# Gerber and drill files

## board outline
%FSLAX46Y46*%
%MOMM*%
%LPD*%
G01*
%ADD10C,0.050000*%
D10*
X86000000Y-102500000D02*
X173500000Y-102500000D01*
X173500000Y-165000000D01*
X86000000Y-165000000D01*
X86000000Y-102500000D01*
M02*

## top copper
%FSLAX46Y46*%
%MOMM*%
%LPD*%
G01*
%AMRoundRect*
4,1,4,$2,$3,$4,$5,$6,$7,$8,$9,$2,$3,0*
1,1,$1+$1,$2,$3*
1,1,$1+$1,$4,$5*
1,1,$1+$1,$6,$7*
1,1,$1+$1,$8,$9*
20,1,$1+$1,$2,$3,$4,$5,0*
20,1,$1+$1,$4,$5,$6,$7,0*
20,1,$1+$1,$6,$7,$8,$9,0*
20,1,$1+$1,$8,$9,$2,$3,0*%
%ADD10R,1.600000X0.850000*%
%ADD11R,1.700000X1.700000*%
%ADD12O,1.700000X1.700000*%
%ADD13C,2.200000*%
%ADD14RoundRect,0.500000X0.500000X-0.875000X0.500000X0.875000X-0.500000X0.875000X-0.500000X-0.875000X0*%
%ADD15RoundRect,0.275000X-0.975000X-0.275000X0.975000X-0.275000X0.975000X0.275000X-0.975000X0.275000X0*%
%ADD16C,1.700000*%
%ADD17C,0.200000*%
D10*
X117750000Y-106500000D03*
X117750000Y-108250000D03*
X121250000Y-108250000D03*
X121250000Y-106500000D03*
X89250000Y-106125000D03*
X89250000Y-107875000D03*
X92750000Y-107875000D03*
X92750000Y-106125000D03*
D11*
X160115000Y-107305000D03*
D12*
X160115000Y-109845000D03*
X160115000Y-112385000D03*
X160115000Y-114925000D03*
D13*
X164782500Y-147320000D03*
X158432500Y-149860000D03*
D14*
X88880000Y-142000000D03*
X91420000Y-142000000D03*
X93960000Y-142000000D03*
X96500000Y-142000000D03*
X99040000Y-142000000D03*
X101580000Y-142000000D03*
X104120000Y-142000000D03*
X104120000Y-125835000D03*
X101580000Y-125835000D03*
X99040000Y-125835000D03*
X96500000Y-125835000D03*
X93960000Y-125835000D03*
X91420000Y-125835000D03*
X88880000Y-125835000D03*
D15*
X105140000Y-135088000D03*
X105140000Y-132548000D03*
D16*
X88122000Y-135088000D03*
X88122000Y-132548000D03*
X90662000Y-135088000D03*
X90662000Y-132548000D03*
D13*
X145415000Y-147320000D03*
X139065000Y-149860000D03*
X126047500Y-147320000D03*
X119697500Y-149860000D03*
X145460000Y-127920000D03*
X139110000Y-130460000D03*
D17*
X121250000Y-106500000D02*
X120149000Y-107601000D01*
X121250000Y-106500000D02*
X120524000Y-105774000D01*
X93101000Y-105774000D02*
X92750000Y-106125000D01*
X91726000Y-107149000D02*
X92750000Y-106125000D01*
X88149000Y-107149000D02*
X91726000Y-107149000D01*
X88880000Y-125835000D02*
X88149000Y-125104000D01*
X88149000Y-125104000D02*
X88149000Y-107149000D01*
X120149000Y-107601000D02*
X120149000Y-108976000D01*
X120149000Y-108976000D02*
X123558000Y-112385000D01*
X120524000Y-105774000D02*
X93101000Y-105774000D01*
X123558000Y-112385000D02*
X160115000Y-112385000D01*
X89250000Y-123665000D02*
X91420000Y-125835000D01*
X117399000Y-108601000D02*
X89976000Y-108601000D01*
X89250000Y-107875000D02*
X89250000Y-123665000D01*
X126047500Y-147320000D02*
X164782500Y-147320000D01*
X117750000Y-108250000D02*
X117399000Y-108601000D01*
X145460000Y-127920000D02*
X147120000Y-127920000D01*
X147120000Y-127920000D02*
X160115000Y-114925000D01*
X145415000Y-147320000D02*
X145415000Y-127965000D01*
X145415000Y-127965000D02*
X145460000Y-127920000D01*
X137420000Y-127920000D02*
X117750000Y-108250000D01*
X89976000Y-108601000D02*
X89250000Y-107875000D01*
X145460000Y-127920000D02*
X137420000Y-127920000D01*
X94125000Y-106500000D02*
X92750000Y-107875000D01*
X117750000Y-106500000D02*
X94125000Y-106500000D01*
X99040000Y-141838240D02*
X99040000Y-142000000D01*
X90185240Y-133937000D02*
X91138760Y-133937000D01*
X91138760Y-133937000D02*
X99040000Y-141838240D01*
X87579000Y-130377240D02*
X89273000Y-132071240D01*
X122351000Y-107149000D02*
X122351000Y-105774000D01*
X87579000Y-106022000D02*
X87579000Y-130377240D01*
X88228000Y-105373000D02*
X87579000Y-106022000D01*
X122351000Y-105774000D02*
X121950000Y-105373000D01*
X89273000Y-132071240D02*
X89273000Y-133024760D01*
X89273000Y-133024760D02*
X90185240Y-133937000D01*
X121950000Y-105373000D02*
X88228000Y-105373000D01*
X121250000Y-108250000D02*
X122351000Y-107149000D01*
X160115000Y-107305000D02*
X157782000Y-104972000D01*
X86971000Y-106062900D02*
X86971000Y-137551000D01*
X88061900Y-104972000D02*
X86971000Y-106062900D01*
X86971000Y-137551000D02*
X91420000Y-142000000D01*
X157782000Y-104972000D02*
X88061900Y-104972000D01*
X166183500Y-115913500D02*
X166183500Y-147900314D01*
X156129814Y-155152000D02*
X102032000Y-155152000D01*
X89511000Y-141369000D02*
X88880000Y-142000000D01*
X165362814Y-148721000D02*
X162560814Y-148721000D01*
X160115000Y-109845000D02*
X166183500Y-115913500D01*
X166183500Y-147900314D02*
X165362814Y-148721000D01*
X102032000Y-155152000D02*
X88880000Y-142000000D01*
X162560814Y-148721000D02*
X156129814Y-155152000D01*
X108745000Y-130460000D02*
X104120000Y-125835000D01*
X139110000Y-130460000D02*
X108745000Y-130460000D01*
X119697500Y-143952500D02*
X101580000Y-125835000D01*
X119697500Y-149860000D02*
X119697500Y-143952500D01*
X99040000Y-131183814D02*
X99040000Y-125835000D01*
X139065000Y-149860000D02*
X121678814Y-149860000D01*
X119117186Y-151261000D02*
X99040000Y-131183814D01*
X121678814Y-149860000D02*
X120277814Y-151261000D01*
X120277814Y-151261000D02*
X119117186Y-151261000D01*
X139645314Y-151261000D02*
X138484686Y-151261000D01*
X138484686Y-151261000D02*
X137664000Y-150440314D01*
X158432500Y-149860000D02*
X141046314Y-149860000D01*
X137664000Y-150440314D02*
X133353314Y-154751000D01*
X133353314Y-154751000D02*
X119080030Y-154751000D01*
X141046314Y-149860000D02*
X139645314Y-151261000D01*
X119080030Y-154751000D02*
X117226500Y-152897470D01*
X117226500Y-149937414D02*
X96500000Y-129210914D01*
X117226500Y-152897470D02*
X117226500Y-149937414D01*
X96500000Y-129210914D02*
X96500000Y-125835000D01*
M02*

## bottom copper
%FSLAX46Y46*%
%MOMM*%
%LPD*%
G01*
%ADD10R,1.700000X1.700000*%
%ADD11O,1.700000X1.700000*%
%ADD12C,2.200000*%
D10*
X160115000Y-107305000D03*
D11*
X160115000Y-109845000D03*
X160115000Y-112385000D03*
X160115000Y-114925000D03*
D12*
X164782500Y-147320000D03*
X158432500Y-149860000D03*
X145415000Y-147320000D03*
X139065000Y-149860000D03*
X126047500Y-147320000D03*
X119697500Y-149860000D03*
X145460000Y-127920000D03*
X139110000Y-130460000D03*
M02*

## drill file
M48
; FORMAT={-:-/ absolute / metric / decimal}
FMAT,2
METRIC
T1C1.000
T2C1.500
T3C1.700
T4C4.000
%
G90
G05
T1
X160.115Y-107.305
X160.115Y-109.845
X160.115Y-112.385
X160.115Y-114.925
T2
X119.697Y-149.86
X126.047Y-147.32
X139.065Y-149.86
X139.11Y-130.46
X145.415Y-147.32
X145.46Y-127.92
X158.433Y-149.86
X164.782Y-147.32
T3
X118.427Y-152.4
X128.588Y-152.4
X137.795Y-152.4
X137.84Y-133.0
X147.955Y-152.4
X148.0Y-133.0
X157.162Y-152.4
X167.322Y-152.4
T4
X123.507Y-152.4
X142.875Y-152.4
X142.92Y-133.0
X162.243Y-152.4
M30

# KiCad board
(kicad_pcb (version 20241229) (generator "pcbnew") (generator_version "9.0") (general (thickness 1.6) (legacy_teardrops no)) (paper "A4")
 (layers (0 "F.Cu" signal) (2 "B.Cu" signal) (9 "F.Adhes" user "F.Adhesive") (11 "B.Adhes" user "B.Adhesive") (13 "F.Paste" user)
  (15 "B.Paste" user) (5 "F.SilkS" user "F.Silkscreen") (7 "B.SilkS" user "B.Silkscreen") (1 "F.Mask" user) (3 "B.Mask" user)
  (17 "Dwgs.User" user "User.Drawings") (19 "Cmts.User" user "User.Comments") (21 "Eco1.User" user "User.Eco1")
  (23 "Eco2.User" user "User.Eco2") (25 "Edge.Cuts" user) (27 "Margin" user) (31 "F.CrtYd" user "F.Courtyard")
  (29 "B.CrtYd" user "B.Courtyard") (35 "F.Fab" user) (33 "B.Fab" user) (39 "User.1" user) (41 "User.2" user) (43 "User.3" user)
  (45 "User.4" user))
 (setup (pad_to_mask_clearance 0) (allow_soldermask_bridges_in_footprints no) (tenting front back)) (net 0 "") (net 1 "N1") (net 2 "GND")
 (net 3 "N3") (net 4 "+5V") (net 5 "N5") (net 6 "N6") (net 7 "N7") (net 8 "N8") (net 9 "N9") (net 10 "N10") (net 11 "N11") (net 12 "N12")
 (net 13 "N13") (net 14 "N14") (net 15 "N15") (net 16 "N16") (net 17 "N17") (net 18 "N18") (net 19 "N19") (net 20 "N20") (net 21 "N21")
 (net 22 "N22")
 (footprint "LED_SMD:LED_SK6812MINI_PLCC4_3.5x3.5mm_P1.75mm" (layer "F.Cu") (at 119.5 107.375)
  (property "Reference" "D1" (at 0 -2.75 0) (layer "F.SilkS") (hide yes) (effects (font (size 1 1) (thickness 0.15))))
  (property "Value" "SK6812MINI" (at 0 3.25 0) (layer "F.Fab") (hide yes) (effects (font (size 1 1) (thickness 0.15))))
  (pad "1" smd rect (at -1.75 -0.875) (size 1.6 0.85) (layers "F.Cu" "F.Mask" "F.Paste") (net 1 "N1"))
  (pad "2" smd rect (at -1.75 0.875) (size 1.6 0.85) (layers "F.Cu" "F.Mask" "F.Paste") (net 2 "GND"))
  (pad "3" smd rect (at 1.75 0.875) (size 1.6 0.85) (layers "F.Cu" "F.Mask" "F.Paste") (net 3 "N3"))
  (pad "4" smd rect (at 1.75 -0.875) (size 1.6 0.85) (layers "F.Cu" "F.Mask" "F.Paste") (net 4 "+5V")))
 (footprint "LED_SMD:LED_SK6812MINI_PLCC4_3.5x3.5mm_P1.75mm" (layer "F.Cu") (at 91 107)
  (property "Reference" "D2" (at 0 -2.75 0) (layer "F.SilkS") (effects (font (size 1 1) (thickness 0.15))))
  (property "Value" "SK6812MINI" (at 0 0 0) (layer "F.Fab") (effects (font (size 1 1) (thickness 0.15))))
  (pad "1" smd rect (at -1.75 -0.875) (size 1.6 0.85) (layers "F.Cu" "F.Mask" "F.Paste") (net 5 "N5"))
  (pad "2" smd rect (at -1.75 0.875) (size 1.6 0.85) (layers "F.Cu" "F.Mask" "F.Paste") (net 2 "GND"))
  (pad "3" smd rect (at 1.75 0.875) (size 1.6 0.85) (layers "F.Cu" "F.Mask" "F.Paste") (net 1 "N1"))
  (pad "4" smd rect (at 1.75 -0.875) (size 1.6 0.85) (layers "F.Cu" "F.Mask" "F.Paste") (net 4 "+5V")))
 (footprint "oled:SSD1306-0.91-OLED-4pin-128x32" (layer "F.Cu") (at 123.615 105.115)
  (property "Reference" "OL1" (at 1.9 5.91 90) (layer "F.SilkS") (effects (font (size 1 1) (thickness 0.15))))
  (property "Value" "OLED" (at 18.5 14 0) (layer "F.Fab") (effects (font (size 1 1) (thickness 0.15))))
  (pad "1" thru_hole rect (at 36.5 2.19) (size 1.7 1.7) (drill 1) (layers "*.Cu" "*.Mask") (remove_unused_layers no) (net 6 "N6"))
  (pad "2" thru_hole oval (at 36.5 4.73) (size 1.7 1.7) (drill 1) (layers "*.Cu" "*.Mask") (remove_unused_layers no) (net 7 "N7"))
  (pad "3" thru_hole oval (at 36.5 7.27) (size 1.7 1.7) (drill 1) (layers "*.Cu" "*.Mask") (remove_unused_layers no) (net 4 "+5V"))
  (pad "4" thru_hole oval (at 36.5 9.81) (size 1.7 1.7) (drill 1) (layers "*.Cu" "*.Mask") (remove_unused_layers no) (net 2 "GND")))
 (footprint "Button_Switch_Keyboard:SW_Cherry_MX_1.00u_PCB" (layer "F.Cu") (at 164.7825 147.32)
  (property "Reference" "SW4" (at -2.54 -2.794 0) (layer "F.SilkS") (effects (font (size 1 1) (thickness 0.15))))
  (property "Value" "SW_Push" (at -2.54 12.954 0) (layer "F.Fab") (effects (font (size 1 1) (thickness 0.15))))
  (pad "" np_thru_hole circle (at -7.62 5.08) (size 1.7 1.7) (drill 1.7) (layers "*.Cu" "*.Mask"))
  (pad "" np_thru_hole circle (at -2.54 5.08) (size 4 4) (drill 4) (layers "*.Cu" "*.Mask"))
  (pad "" np_thru_hole circle (at 2.54 5.08) (size 1.7 1.7) (drill 1.7) (layers "*.Cu" "*.Mask"))
  (pad "1" thru_hole circle (at 0 0) (size 2.2 2.2) (drill 1.5) (layers "*.Cu" "*.Mask") (remove_unused_layers no) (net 2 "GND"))
  (pad "2" thru_hole circle (at -6.35 2.54) (size 2.2 2.2) (drill 1.5) (layers "*.Cu" "*.Mask") (remove_unused_layers no) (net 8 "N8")))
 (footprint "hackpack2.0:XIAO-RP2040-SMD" (layer "F.Cu") (at 96.5 134 90)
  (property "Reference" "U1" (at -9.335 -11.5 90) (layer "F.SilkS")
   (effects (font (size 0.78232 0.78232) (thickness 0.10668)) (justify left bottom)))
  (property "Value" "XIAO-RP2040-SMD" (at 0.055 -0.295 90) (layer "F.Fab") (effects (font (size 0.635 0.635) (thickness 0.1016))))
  (pad "1" smd roundrect (at -8 -7.62 90) (size 2.75 2) (layers "F.Cu" "F.Mask" "F.Paste") (roundrect_rratio 0.25) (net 7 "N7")
   (solder_mask_margin 0.0508) (thermal_bridge_angle 45))
  (pad "2" smd roundrect (at -8 -5.08 90) (size 2.75 2) (layers "F.Cu" "F.Mask" "F.Paste") (roundrect_rratio 0.25) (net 6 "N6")
   (solder_mask_margin 0.0508) (thermal_bridge_angle 45))
  (pad "3" smd roundrect (at -8 -2.54 90) (size 2.75 2) (layers "F.Cu" "F.Mask" "F.Paste") (roundrect_rratio 0.25) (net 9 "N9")
   (solder_mask_margin 0.0508) (thermal_bridge_angle 45))
  (pad "4" smd roundrect (at -8 0 90) (size 2.75 2) (layers "F.Cu" "F.Mask" "F.Paste") (roundrect_rratio 0.25) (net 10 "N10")
   (solder_mask_margin 0.0508) (thermal_bridge_angle 45))
  (pad "5" smd roundrect (at -8 2.54 90) (size 2.75 2) (layers "F.Cu" "F.Mask" "F.Paste") (roundrect_rratio 0.25) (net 3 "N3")
   (solder_mask_margin 0.0508) (thermal_bridge_angle 45))
  (pad "6" smd roundrect (at -8 5.08 90) (size 2.75 2) (layers "F.Cu" "F.Mask" "F.Paste") (roundrect_rratio 0.25) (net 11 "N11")
   (solder_mask_margin 0.0508) (thermal_bridge_angle 45))
  (pad "7" smd roundrect (at -8 7.62 90) (size 2.75 2) (layers "F.Cu" "F.Mask" "F.Paste") (roundrect_rratio 0.25) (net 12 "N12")
   (solder_mask_margin 0.0508) (thermal_bridge_angle 45))
  (pad "8" smd roundrect (at 8.165 7.62 90) (size 2.75 2) (layers "F.Cu" "F.Mask" "F.Paste") (roundrect_rratio 0.25) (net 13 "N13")
   (solder_mask_margin 0.0508) (thermal_bridge_angle 45))
  (pad "9" smd roundrect (at 8.165 5.08 90) (size 2.75 2) (layers "F.Cu" "F.Mask" "F.Paste") (roundrect_rratio 0.25) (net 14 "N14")
   (solder_mask_margin 0.0508) (thermal_bridge_angle 45))
  (pad "10" smd roundrect (at 8.165 2.54 90) (size 2.75 2) (layers "F.Cu" "F.Mask" "F.Paste") (roundrect_rratio 0.25) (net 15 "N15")
   (solder_mask_margin 0.0508) (thermal_bridge_angle 45))
  (pad "11" smd roundrect (at 8.165 0 90) (size 2.75 2) (layers "F.Cu" "F.Mask" "F.Paste") (roundrect_rratio 0.25) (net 8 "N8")
   (solder_mask_margin 0.0508) (thermal_bridge_angle 45))
  (pad "12" smd roundrect (at 8.165 -2.54 90) (size 2.75 2) (layers "F.Cu" "F.Mask" "F.Paste") (roundrect_rratio 0.25) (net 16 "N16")
   (solder_mask_margin 0.0508) (thermal_bridge_angle 45))
  (pad "13" smd roundrect (at 8.165 -5.08 90) (size 2.75 2) (layers "F.Cu" "F.Mask" "F.Paste") (roundrect_rratio 0.25) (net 2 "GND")
   (solder_mask_margin 0.0508) (thermal_bridge_angle 45))
  (pad "14" smd roundrect (at 8.165 -7.62 90) (size 2.75 2) (layers "F.Cu" "F.Mask" "F.Paste") (roundrect_rratio 0.25) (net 4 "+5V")
   (solder_mask_margin 0.0508) (thermal_bridge_angle 45))
  (pad "15" smd roundrect (at -1.088 8.64) (size 2.5 1.1) (layers "F.Cu" "F.Mask" "F.Paste") (roundrect_rratio 0.25) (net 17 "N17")
   (thermal_bridge_angle 45))
  (pad "16" smd roundrect (at 1.452 8.64) (size 2.5 1.1) (layers "F.Cu" "F.Mask" "F.Paste") (roundrect_rratio 0.25) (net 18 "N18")
   (thermal_bridge_angle 45))
  (pad "17" smd circle (at -1.088 -8.378 90) (size 1.7 1.7) (layers "F.Cu" "F.Mask" "F.Paste") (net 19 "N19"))
  (pad "18" smd circle (at 1.452 -8.378 90) (size 1.7 1.7) (layers "F.Cu" "F.Mask" "F.Paste") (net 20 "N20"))
  (pad "19" smd circle (at -1.088 -5.838 90) (size 1.7 1.7) (layers "F.Cu" "F.Mask" "F.Paste") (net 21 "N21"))
  (pad "20" smd circle (at 1.452 -5.838 90) (size 1.7 1.7) (layers "F.Cu" "F.Mask" "F.Paste") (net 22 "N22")))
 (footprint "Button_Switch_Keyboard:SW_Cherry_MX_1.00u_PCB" (layer "F.Cu") (at 145.415 147.32)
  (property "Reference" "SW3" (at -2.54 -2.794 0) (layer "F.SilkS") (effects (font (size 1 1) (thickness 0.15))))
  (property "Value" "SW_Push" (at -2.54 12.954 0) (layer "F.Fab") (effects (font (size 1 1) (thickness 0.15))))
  (pad "" np_thru_hole circle (at -7.62 5.08) (size 1.7 1.7) (drill 1.7) (layers "*.Cu" "*.Mask"))
  (pad "" np_thru_hole circle (at -2.54 5.08) (size 4 4) (drill 4) (layers "*.Cu" "*.Mask"))
  (pad "" np_thru_hole circle (at 2.54 5.08) (size 1.7 1.7) (drill 1.7) (layers "*.Cu" "*.Mask"))
  (pad "1" thru_hole circle (at 0 0) (size 2.2 2.2) (drill 1.5) (layers "*.Cu" "*.Mask") (remove_unused_layers no) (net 2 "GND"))
  (pad "2" thru_hole circle (at -6.35 2.54) (size 2.2 2.2) (drill 1.5) (layers "*.Cu" "*.Mask") (remove_unused_layers no) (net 15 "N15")))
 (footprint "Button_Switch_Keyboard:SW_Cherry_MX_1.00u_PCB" (layer "F.Cu") (at 126.0475 147.32)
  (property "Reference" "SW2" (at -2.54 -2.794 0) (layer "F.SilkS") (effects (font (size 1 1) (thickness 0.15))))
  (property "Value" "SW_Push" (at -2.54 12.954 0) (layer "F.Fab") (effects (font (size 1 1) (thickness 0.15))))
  (pad "" np_thru_hole circle (at -7.62 5.08) (size 1.7 1.7) (drill 1.7) (layers "*.Cu" "*.Mask"))
  (pad "" np_thru_hole circle (at -2.54 5.08) (size 4 4) (drill 4) (layers "*.Cu" "*.Mask"))
  (pad "" np_thru_hole circle (at 2.54 5.08) (size 1.7 1.7) (drill 1.7) (layers "*.Cu" "*.Mask"))
  (pad "1" thru_hole circle (at 0 0) (size 2.2 2.2) (drill 1.5) (layers "*.Cu" "*.Mask") (remove_unused_layers no) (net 2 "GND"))
  (pad "2" thru_hole circle (at -6.35 2.54) (size 2.2 2.2) (drill 1.5) (layers "*.Cu" "*.Mask") (remove_unused_layers no) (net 14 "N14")))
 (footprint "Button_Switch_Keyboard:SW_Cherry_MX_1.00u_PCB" (layer "F.Cu") (at 145.46 127.92)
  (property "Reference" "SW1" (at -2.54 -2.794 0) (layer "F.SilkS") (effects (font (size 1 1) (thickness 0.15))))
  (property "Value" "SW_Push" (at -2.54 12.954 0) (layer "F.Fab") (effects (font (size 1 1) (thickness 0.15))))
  (pad "" np_thru_hole circle (at -7.62 5.08) (size 1.7 1.7) (drill 1.7) (layers "*.Cu" "*.Mask"))
  (pad "" np_thru_hole circle (at -2.54 5.08) (size 4 4) (drill 4) (layers "*.Cu" "*.Mask"))
  (pad "" np_thru_hole circle (at 2.54 5.08) (size 1.7 1.7) (drill 1.7) (layers "*.Cu" "*.Mask"))
  (pad "1" thru_hole circle (at 0 0) (size 2.2 2.2) (drill 1.5) (layers "*.Cu" "*.Mask") (remove_unused_layers no) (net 2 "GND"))
  (pad "2" thru_hole circle (at -6.35 2.54) (size 2.2 2.2) (drill 1.5) (layers "*.Cu" "*.Mask") (remove_unused_layers no) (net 13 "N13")))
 (gr_rect (start 86 102.5) (end 173.5 165) (stroke (width 0.05) (type default)) (fill no) (layer "Edge.Cuts"))
 (segment (start 121.25 106.5) (end 120.149 107.601) (width 0.2) (layer "F.Cu") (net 4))
 (segment (start 121.25 106.5) (end 120.524 105.774) (width 0.2) (layer "F.Cu") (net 4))
 (segment (start 93.101 105.774) (end 92.75 106.125) (width 0.2) (layer "F.Cu") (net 4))
 (segment (start 91.726 107.149) (end 92.75 106.125) (width 0.2) (layer "F.Cu") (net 4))
 (segment (start 88.149 107.149) (end 91.726 107.149) (width 0.2) (layer "F.Cu") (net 4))
 (segment (start 88.88 125.835) (end 88.149 125.104) (width 0.2) (layer "F.Cu") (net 4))
 (segment (start 88.149 125.104) (end 88.149 107.149) (width 0.2) (layer "F.Cu") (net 4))
 (segment (start 120.149 107.601) (end 120.149 108.976) (width 0.2) (layer "F.Cu") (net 4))
 (segment (start 120.149 108.976) (end 123.558 112.385) (width 0.2) (layer "F.Cu") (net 4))
 (segment (start 120.524 105.774) (end 93.101 105.774) (width 0.2) (layer "F.Cu") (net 4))
 (segment (start 123.558 112.385) (end 160.115 112.385) (width 0.2) (layer "F.Cu") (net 4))
 (segment (start 89.25 123.665) (end 91.42 125.835) (width 0.2) (layer "F.Cu") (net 2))
 (segment (start 117.399 108.601) (end 89.976 108.601) (width 0.2) (layer "F.Cu") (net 2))
 (segment (start 89.25 107.875) (end 89.25 123.665) (width 0.2) (layer "F.Cu") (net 2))
 (segment (start 126.0475 147.32) (end 164.7825 147.32) (width 0.2) (layer "F.Cu") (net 2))
 (segment (start 117.75 108.25) (end 117.399 108.601) (width 0.2) (layer "F.Cu") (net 2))
 (segment (start 145.46 127.92) (end 147.12 127.92) (width 0.2) (layer "F.Cu") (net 2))
 (segment (start 147.12 127.92) (end 160.115 114.925) (width 0.2) (layer "F.Cu") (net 2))
 (segment (start 145.415 147.32) (end 145.415 127.965) (width 0.2) (layer "F.Cu") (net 2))
 (segment (start 145.415 127.965) (end 145.46 127.92) (width 0.2) (layer "F.Cu") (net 2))
 (segment (start 137.42 127.92) (end 117.75 108.25) (width 0.2) (layer "F.Cu") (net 2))
 (segment (start 89.976 108.601) (end 89.25 107.875) (width 0.2) (layer "F.Cu") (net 2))
 (segment (start 145.46 127.92) (end 137.42 127.92) (width 0.2) (layer "F.Cu") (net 2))
 (segment (start 94.125 106.5) (end 92.75 107.875) (width 0.2) (layer "F.Cu") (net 1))
 (segment (start 117.75 106.5) (end 94.125 106.5) (width 0.2) (layer "F.Cu") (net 1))
 (segment (start 99.04 141.83824) (end 99.04 142) (width 0.2) (layer "F.Cu") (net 3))
 (segment (start 90.18524 133.937) (end 91.13876 133.937) (width 0.2) (layer "F.Cu") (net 3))
 (segment (start 91.13876 133.937) (end 99.04 141.83824) (width 0.2) (layer "F.Cu") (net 3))
 (segment (start 87.579 130.37724) (end 89.273 132.07124) (width 0.2) (layer "F.Cu") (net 3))
 (segment (start 122.351 107.149) (end 122.351 105.774) (width 0.2) (layer "F.Cu") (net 3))
 (segment (start 87.579 106.022) (end 87.579 130.37724) (width 0.2) (layer "F.Cu") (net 3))
 (segment (start 88.228 105.373) (end 87.579 106.022) (width 0.2) (layer "F.Cu") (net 3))
 (segment (start 122.351 105.774) (end 121.95 105.373) (width 0.2) (layer "F.Cu") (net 3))
 (segment (start 89.273 132.07124) (end 89.273 133.02476) (width 0.2) (layer "F.Cu") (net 3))
 (segment (start 89.273 133.02476) (end 90.18524 133.937) (width 0.2) (layer "F.Cu") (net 3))
 (segment (start 121.95 105.373) (end 88.228 105.373) (width 0.2) (layer "F.Cu") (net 3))
 (segment (start 121.25 108.25) (end 122.351 107.149) (width 0.2) (layer "F.Cu") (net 3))
 (segment (start 160.115 107.305) (end 157.782 104.972) (width 0.2) (layer "F.Cu") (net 6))
 (segment (start 86.971 106.0629) (end 86.971 137.551) (width 0.2) (layer "F.Cu") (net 6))
 (segment (start 88.0619 104.972) (end 86.971 106.0629) (width 0.2) (layer "F.Cu") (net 6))
 (segment (start 86.971 137.551) (end 91.42 142) (width 0.2) (layer "F.Cu") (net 6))
 (segment (start 157.782 104.972) (end 88.0619 104.972) (width 0.2) (layer "F.Cu") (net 6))
 (segment (start 166.1835 115.9135) (end 166.1835 147.900314) (width 0.2) (layer "F.Cu") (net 7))
 (segment (start 156.129814 155.152) (end 102.032 155.152) (width 0.2) (layer "F.Cu") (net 7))
 (segment (start 89.511 141.369) (end 88.88 142) (width 0.2) (layer "F.Cu") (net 7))
 (segment (start 165.362814 148.721) (end 162.560814 148.721) (width 0.2) (layer "F.Cu") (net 7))
 (segment (start 160.115 109.845) (end 166.1835 115.9135) (width 0.2) (layer "F.Cu") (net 7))
 (segment (start 166.1835 147.900314) (end 165.362814 148.721) (width 0.2) (layer "F.Cu") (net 7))
 (segment (start 102.032 155.152) (end 88.88 142) (width 0.2) (layer "F.Cu") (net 7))
 (segment (start 162.560814 148.721) (end 156.129814 155.152) (width 0.2) (layer "F.Cu") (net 7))
 (segment (start 108.745 130.46) (end 104.12 125.835) (width 0.2) (layer "F.Cu") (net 13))
 (segment (start 139.11 130.46) (end 108.745 130.46) (width 0.2) (layer "F.Cu") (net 13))
 (segment (start 119.6975 143.9525) (end 101.58 125.835) (width 0.2) (layer "F.Cu") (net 14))
 (segment (start 119.6975 149.86) (end 119.6975 143.9525) (width 0.2) (layer "F.Cu") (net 14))
 (segment (start 99.04 131.183814) (end 99.04 125.835) (width 0.2) (layer "F.Cu") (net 15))
 (segment (start 139.065 149.86) (end 121.678814 149.86) (width 0.2) (layer "F.Cu") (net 15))
 (segment (start 119.117186 151.261) (end 99.04 131.183814) (width 0.2) (layer "F.Cu") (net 15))
 (segment (start 121.678814 149.86) (end 120.277814 151.261) (width 0.2) (layer "F.Cu") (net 15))
 (segment (start 120.277814 151.261) (end 119.117186 151.261) (width 0.2) (layer "F.Cu") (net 15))
 (segment (start 139.645314 151.261) (end 138.484686 151.261) (width 0.2) (layer "F.Cu") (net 8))
 (segment (start 138.484686 151.261) (end 137.664 150.440314) (width 0.2) (layer "F.Cu") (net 8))
 (segment (start 158.4325 149.86) (end 141.046314 149.86) (width 0.2) (layer "F.Cu") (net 8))
 (segment (start 137.664 150.440314) (end 133.353314 154.751) (width 0.2) (layer "F.Cu") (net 8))
 (segment (start 133.353314 154.751) (end 119.08003 154.751) (width 0.2) (layer "F.Cu") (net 8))
 (segment (start 141.046314 149.86) (end 139.645314 151.261) (width 0.2) (layer "F.Cu") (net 8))
 (segment (start 119.08003 154.751) (end 117.2265 152.89747) (width 0.2) (layer "F.Cu") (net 8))
 (segment (start 117.2265 149.937414) (end 96.5 129.210914) (width 0.2) (layer "F.Cu") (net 8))
 (segment (start 117.2265 152.89747) (end 117.2265 149.937414) (width 0.2) (layer "F.Cu") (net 8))
 (segment (start 96.5 129.210914) (end 96.5 125.835) (width 0.2) (layer "F.Cu") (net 8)))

